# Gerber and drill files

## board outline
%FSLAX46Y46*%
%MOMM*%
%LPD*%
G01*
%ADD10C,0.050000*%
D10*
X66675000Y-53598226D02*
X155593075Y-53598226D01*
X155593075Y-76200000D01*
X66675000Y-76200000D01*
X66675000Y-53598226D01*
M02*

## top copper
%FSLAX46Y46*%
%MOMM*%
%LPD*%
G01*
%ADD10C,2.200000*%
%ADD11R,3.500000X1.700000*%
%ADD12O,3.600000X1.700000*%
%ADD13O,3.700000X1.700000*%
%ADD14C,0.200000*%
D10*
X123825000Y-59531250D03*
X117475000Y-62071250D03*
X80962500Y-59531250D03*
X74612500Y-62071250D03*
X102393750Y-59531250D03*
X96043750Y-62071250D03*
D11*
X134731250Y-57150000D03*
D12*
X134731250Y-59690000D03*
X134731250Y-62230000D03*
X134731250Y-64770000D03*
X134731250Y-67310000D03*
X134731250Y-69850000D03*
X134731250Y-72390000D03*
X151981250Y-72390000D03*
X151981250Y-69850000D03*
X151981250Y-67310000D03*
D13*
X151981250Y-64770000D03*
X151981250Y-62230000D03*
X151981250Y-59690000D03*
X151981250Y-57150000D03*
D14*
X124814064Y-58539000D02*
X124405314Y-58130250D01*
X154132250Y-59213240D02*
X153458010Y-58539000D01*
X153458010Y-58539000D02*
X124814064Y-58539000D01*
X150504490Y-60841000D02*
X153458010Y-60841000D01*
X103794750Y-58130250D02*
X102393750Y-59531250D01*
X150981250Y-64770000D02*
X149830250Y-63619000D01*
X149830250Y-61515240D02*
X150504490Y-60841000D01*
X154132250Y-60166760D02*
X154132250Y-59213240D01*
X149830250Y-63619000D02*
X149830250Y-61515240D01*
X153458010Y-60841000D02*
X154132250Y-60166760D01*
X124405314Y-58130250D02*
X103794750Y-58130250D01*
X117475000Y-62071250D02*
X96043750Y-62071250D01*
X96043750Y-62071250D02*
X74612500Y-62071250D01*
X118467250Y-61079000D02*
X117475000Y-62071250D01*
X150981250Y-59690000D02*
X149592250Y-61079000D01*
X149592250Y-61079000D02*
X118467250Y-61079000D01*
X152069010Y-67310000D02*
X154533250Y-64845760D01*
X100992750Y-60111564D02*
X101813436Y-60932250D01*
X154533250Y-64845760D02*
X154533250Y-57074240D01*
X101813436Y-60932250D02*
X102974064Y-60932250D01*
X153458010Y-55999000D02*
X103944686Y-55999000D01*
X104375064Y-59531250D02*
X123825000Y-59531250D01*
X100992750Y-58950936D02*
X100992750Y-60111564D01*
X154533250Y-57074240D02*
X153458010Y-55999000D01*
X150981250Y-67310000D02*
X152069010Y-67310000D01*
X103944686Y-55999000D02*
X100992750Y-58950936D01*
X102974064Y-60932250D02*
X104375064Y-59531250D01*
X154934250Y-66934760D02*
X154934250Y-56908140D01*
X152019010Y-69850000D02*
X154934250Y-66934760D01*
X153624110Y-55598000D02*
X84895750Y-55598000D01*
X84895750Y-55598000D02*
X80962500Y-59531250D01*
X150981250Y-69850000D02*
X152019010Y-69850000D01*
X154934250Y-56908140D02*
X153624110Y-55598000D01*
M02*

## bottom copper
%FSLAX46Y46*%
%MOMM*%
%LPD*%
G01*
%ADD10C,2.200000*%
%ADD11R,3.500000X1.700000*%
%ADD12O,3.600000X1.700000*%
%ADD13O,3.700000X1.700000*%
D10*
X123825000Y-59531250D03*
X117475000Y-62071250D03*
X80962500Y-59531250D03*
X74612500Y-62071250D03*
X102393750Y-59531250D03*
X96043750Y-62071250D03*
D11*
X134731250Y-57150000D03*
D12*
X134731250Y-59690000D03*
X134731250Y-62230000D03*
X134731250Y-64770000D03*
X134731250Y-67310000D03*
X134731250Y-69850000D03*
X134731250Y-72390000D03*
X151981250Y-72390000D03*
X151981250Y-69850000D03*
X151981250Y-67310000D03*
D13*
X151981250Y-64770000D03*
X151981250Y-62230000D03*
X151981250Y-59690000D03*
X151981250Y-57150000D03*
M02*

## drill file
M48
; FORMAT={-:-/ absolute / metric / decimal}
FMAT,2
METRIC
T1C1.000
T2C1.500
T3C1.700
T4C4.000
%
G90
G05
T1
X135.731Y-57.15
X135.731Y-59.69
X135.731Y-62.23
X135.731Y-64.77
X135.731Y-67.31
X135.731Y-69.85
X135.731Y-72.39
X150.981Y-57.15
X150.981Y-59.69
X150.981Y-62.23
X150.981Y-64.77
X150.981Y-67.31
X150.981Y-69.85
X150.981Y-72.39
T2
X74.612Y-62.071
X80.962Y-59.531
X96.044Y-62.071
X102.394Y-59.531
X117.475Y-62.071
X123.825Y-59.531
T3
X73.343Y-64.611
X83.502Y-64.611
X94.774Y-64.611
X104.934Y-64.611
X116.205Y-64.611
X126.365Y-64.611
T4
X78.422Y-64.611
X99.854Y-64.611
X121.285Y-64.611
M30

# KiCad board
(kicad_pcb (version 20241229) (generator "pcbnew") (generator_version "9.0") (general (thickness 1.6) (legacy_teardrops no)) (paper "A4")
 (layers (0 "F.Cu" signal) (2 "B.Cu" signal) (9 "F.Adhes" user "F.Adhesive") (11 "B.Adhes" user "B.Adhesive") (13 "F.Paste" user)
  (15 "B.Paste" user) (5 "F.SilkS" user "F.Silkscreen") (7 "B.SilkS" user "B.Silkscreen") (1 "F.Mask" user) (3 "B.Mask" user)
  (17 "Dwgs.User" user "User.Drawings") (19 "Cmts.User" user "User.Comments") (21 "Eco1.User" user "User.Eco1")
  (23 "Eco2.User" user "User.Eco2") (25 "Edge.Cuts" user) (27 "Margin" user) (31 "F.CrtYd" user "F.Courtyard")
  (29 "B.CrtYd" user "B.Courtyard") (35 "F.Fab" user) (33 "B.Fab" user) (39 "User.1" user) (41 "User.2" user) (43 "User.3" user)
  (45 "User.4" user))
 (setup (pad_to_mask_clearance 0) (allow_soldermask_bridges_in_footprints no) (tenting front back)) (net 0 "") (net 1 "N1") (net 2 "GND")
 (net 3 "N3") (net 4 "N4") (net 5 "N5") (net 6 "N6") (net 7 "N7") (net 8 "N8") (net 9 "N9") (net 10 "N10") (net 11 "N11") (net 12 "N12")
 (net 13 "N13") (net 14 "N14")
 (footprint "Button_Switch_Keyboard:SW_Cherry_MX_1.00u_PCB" (layer "F.Cu") (at 123.825 59.53125)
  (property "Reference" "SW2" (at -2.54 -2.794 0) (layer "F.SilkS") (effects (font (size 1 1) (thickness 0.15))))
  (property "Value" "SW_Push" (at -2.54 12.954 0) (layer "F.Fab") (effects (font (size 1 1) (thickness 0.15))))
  (pad "" np_thru_hole circle (at -7.62 5.08) (size 1.7 1.7) (drill 1.7) (layers "*.Cu" "*.Mask"))
  (pad "" np_thru_hole circle (at -2.54 5.08) (size 4 4) (drill 4) (layers "*.Cu" "*.Mask"))
  (pad "" np_thru_hole circle (at 2.54 5.08) (size 1.7 1.7) (drill 1.7) (layers "*.Cu" "*.Mask"))
  (pad "1" thru_hole circle (at 0 0) (size 2.2 2.2) (drill 1.5) (layers "*.Cu" "*.Mask") (remove_unused_layers no) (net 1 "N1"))
  (pad "2" thru_hole circle (at -6.35 2.54) (size 2.2 2.2) (drill 1.5) (layers "*.Cu" "*.Mask") (remove_unused_layers no) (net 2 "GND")))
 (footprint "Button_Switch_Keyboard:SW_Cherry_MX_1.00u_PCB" (layer "F.Cu") (at 80.9625 59.53125)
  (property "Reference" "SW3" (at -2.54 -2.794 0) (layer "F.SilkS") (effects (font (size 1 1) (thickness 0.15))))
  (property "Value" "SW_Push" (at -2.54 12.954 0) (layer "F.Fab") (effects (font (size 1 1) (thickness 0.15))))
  (pad "" np_thru_hole circle (at -7.62 5.08) (size 1.7 1.7) (drill 1.7) (layers "*.Cu" "*.Mask"))
  (pad "" np_thru_hole circle (at -2.54 5.08) (size 4 4) (drill 4) (layers "*.Cu" "*.Mask"))
  (pad "" np_thru_hole circle (at 2.54 5.08) (size 1.7 1.7) (drill 1.7) (layers "*.Cu" "*.Mask"))
  (pad "1" thru_hole circle (at 0 0) (size 2.2 2.2) (drill 1.5) (layers "*.Cu" "*.Mask") (remove_unused_layers no) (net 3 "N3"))
  (pad "2" thru_hole circle (at -6.35 2.54) (size 2.2 2.2) (drill 1.5) (layers "*.Cu" "*.Mask") (remove_unused_layers no) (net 2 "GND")))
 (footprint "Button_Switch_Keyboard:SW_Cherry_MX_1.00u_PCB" (layer "F.Cu") (at 102.39375 59.53125)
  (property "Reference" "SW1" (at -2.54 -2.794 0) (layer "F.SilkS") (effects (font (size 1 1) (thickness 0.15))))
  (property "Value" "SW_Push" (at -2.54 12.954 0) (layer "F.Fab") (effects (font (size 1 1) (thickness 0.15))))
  (pad "" np_thru_hole circle (at -7.62 5.08) (size 1.7 1.7) (drill 1.7) (layers "*.Cu" "*.Mask"))
  (pad "" np_thru_hole circle (at -2.54 5.08) (size 4 4) (drill 4) (layers "*.Cu" "*.Mask"))
  (pad "" np_thru_hole circle (at 2.54 5.08) (size 1.7 1.7) (drill 1.7) (layers "*.Cu" "*.Mask"))
  (pad "1" thru_hole circle (at 0 0) (size 2.2 2.2) (drill 1.5) (layers "*.Cu" "*.Mask") (remove_unused_layers no) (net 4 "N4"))
  (pad "2" thru_hole circle (at -6.35 2.54) (size 2.2 2.2) (drill 1.5) (layers "*.Cu" "*.Mask") (remove_unused_layers no) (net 2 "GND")))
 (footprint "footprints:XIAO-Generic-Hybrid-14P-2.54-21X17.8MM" (layer "F.Cu") (at 143.35625 64.77)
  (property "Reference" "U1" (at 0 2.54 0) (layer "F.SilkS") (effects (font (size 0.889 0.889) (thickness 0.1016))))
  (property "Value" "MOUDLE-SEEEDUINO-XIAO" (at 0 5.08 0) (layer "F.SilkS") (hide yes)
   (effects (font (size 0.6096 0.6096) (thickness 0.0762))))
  (pad "1" thru_hole rect (at -7.625 -7.62) (size 3.5 1.7) (drill 1 (offset -1 0)) (layers "*.Cu" "*.Mask") (remove_unused_layers no)
   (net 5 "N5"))
  (pad "2" thru_hole oval (at -7.625 -5.08) (size 3.6 1.7) (drill 1 (offset -1 0)) (layers "*.Cu" "*.Mask") (remove_unused_layers no)
   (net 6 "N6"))
  (pad "3" thru_hole oval (at -7.625 -2.54) (size 3.6 1.7) (drill 1 (offset -1 0)) (layers "*.Cu" "*.Mask") (remove_unused_layers no)
   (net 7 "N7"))
  (pad "4" thru_hole oval (at -7.625 0) (size 3.6 1.7) (drill 1 (offset -1 0)) (layers "*.Cu" "*.Mask") (remove_unused_layers no)
   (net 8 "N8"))
  (pad "5" thru_hole oval (at -7.625 2.54) (size 3.6 1.7) (drill 1 (offset -1 0)) (layers "*.Cu" "*.Mask") (remove_unused_layers no)
   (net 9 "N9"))
  (pad "6" thru_hole oval (at -7.625 5.08 180) (size 3.6 1.7) (drill 1 (offset 1 0)) (layers "*.Cu" "*.Mask") (remove_unused_layers no)
   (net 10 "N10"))
  (pad "7" thru_hole oval (at -7.625 7.62) (size 3.6 1.7) (drill 1 (offset -1 0)) (layers "*.Cu" "*.Mask") (remove_unused_layers no)
   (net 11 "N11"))
  (pad "8" thru_hole oval (at 7.625 7.62) (size 3.6 1.7) (drill 1 (offset 1 0)) (layers "*.Cu" "*.Mask") (remove_unused_layers no)
   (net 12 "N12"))
  (pad "9" thru_hole oval (at 7.625 5.08) (size 3.6 1.7) (drill 1 (offset 1 0)) (layers "*.Cu" "*.Mask") (remove_unused_layers no)
   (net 3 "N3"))
  (pad "10" thru_hole oval (at 7.625 2.54) (size 3.6 1.7) (drill 1 (offset 1 0)) (layers "*.Cu" "*.Mask") (remove_unused_layers no)
   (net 1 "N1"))
  (pad "11" thru_hole oval (at 7.625 0) (size 3.7 1.7) (drill 1 (offset 1 0)) (layers "*.Cu" "*.Mask") (remove_unused_layers no)
   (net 4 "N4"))
  (pad "12" thru_hole oval (at 7.625 -2.54) (size 3.7 1.7) (drill 1 (offset 1 0)) (layers "*.Cu" "*.Mask") (remove_unused_layers no)
   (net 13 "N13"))
  (pad "13" thru_hole oval (at 7.625 -5.08) (size 3.7 1.7) (drill 1 (offset 1 0)) (layers "*.Cu" "*.Mask") (remove_unused_layers no)
   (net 2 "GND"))
  (pad "14" thru_hole oval (at 7.625 -7.62) (size 3.7 1.7) (drill 1 (offset 1 0)) (layers "*.Cu" "*.Mask") (remove_unused_layers no)
   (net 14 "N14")))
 (gr_rect (start 66.675 53.598226) (end 155.593075 76.2) (stroke (width 0.05) (type default)) (fill no) (layer "Edge.Cuts"))
 (segment (start 124.814064 58.539) (end 124.405314 58.13025) (width 0.2) (layer "F.Cu") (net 4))
 (segment (start 154.13225 59.21324) (end 153.45801 58.539) (width 0.2) (layer "F.Cu") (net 4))
 (segment (start 153.45801 58.539) (end 124.814064 58.539) (width 0.2) (layer "F.Cu") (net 4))
 (segment (start 150.50449 60.841) (end 153.45801 60.841) (width 0.2) (layer "F.Cu") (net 4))
 (segment (start 103.79475 58.13025) (end 102.39375 59.53125) (width 0.2) (layer "F.Cu") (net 4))
 (segment (start 150.98125 64.77) (end 149.83025 63.619) (width 0.2) (layer "F.Cu") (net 4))
 (segment (start 149.83025 61.51524) (end 150.50449 60.841) (width 0.2) (layer "F.Cu") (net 4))
 (segment (start 154.13225 60.16676) (end 154.13225 59.21324) (width 0.2) (layer "F.Cu") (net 4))
 (segment (start 149.83025 63.619) (end 149.83025 61.51524) (width 0.2) (layer "F.Cu") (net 4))
 (segment (start 153.45801 60.841) (end 154.13225 60.16676) (width 0.2) (layer "F.Cu") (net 4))
 (segment (start 124.405314 58.13025) (end 103.79475 58.13025) (width 0.2) (layer "F.Cu") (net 4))
 (segment (start 117.475 62.07125) (end 96.04375 62.07125) (width 0.2) (layer "F.Cu") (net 2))
 (segment (start 96.04375 62.07125) (end 74.6125 62.07125) (width 0.2) (layer "F.Cu") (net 2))
 (segment (start 118.46725 61.079) (end 117.475 62.07125) (width 0.2) (layer "F.Cu") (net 2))
 (segment (start 150.98125 59.69) (end 149.59225 61.079) (width 0.2) (layer "F.Cu") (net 2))
 (segment (start 149.59225 61.079) (end 118.46725 61.079) (width 0.2) (layer "F.Cu") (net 2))
 (segment (start 152.06901 67.31) (end 154.53325 64.84576) (width 0.2) (layer "F.Cu") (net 1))
 (segment (start 100.99275 60.111564) (end 101.813436 60.93225) (width 0.2) (layer "F.Cu") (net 1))
 (segment (start 154.53325 64.84576) (end 154.53325 57.07424) (width 0.2) (layer "F.Cu") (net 1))
 (segment (start 101.813436 60.93225) (end 102.974064 60.93225) (width 0.2) (layer "F.Cu") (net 1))
 (segment (start 153.45801 55.999) (end 103.944686 55.999) (width 0.2) (layer "F.Cu") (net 1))
 (segment (start 104.375064 59.53125) (end 123.825 59.53125) (width 0.2) (layer "F.Cu") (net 1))
 (segment (start 100.99275 58.950936) (end 100.99275 60.111564) (width 0.2) (layer "F.Cu") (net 1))
 (segment (start 154.53325 57.07424) (end 153.45801 55.999) (width 0.2) (layer "F.Cu") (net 1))
 (segment (start 150.98125 67.31) (end 152.06901 67.31) (width 0.2) (layer "F.Cu") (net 1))
 (segment (start 103.944686 55.999) (end 100.99275 58.950936) (width 0.2) (layer "F.Cu") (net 1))
 (segment (start 102.974064 60.93225) (end 104.375064 59.53125) (width 0.2) (layer "F.Cu") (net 1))
 (segment (start 154.93425 66.93476) (end 154.93425 56.90814) (width 0.2) (layer "F.Cu") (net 3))
 (segment (start 152.01901 69.85) (end 154.93425 66.93476) (width 0.2) (layer "F.Cu") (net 3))
 (segment (start 153.62411 55.598) (end 84.89575 55.598) (width 0.2) (layer "F.Cu") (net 3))
 (segment (start 84.89575 55.598) (end 80.9625 59.53125) (width 0.2) (layer "F.Cu") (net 3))
 (segment (start 150.98125 69.85) (end 152.01901 69.85) (width 0.2) (layer "F.Cu") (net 3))
 (segment (start 154.93425 56.90814) (end 153.62411 55.598) (width 0.2) (layer "F.Cu") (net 3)))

